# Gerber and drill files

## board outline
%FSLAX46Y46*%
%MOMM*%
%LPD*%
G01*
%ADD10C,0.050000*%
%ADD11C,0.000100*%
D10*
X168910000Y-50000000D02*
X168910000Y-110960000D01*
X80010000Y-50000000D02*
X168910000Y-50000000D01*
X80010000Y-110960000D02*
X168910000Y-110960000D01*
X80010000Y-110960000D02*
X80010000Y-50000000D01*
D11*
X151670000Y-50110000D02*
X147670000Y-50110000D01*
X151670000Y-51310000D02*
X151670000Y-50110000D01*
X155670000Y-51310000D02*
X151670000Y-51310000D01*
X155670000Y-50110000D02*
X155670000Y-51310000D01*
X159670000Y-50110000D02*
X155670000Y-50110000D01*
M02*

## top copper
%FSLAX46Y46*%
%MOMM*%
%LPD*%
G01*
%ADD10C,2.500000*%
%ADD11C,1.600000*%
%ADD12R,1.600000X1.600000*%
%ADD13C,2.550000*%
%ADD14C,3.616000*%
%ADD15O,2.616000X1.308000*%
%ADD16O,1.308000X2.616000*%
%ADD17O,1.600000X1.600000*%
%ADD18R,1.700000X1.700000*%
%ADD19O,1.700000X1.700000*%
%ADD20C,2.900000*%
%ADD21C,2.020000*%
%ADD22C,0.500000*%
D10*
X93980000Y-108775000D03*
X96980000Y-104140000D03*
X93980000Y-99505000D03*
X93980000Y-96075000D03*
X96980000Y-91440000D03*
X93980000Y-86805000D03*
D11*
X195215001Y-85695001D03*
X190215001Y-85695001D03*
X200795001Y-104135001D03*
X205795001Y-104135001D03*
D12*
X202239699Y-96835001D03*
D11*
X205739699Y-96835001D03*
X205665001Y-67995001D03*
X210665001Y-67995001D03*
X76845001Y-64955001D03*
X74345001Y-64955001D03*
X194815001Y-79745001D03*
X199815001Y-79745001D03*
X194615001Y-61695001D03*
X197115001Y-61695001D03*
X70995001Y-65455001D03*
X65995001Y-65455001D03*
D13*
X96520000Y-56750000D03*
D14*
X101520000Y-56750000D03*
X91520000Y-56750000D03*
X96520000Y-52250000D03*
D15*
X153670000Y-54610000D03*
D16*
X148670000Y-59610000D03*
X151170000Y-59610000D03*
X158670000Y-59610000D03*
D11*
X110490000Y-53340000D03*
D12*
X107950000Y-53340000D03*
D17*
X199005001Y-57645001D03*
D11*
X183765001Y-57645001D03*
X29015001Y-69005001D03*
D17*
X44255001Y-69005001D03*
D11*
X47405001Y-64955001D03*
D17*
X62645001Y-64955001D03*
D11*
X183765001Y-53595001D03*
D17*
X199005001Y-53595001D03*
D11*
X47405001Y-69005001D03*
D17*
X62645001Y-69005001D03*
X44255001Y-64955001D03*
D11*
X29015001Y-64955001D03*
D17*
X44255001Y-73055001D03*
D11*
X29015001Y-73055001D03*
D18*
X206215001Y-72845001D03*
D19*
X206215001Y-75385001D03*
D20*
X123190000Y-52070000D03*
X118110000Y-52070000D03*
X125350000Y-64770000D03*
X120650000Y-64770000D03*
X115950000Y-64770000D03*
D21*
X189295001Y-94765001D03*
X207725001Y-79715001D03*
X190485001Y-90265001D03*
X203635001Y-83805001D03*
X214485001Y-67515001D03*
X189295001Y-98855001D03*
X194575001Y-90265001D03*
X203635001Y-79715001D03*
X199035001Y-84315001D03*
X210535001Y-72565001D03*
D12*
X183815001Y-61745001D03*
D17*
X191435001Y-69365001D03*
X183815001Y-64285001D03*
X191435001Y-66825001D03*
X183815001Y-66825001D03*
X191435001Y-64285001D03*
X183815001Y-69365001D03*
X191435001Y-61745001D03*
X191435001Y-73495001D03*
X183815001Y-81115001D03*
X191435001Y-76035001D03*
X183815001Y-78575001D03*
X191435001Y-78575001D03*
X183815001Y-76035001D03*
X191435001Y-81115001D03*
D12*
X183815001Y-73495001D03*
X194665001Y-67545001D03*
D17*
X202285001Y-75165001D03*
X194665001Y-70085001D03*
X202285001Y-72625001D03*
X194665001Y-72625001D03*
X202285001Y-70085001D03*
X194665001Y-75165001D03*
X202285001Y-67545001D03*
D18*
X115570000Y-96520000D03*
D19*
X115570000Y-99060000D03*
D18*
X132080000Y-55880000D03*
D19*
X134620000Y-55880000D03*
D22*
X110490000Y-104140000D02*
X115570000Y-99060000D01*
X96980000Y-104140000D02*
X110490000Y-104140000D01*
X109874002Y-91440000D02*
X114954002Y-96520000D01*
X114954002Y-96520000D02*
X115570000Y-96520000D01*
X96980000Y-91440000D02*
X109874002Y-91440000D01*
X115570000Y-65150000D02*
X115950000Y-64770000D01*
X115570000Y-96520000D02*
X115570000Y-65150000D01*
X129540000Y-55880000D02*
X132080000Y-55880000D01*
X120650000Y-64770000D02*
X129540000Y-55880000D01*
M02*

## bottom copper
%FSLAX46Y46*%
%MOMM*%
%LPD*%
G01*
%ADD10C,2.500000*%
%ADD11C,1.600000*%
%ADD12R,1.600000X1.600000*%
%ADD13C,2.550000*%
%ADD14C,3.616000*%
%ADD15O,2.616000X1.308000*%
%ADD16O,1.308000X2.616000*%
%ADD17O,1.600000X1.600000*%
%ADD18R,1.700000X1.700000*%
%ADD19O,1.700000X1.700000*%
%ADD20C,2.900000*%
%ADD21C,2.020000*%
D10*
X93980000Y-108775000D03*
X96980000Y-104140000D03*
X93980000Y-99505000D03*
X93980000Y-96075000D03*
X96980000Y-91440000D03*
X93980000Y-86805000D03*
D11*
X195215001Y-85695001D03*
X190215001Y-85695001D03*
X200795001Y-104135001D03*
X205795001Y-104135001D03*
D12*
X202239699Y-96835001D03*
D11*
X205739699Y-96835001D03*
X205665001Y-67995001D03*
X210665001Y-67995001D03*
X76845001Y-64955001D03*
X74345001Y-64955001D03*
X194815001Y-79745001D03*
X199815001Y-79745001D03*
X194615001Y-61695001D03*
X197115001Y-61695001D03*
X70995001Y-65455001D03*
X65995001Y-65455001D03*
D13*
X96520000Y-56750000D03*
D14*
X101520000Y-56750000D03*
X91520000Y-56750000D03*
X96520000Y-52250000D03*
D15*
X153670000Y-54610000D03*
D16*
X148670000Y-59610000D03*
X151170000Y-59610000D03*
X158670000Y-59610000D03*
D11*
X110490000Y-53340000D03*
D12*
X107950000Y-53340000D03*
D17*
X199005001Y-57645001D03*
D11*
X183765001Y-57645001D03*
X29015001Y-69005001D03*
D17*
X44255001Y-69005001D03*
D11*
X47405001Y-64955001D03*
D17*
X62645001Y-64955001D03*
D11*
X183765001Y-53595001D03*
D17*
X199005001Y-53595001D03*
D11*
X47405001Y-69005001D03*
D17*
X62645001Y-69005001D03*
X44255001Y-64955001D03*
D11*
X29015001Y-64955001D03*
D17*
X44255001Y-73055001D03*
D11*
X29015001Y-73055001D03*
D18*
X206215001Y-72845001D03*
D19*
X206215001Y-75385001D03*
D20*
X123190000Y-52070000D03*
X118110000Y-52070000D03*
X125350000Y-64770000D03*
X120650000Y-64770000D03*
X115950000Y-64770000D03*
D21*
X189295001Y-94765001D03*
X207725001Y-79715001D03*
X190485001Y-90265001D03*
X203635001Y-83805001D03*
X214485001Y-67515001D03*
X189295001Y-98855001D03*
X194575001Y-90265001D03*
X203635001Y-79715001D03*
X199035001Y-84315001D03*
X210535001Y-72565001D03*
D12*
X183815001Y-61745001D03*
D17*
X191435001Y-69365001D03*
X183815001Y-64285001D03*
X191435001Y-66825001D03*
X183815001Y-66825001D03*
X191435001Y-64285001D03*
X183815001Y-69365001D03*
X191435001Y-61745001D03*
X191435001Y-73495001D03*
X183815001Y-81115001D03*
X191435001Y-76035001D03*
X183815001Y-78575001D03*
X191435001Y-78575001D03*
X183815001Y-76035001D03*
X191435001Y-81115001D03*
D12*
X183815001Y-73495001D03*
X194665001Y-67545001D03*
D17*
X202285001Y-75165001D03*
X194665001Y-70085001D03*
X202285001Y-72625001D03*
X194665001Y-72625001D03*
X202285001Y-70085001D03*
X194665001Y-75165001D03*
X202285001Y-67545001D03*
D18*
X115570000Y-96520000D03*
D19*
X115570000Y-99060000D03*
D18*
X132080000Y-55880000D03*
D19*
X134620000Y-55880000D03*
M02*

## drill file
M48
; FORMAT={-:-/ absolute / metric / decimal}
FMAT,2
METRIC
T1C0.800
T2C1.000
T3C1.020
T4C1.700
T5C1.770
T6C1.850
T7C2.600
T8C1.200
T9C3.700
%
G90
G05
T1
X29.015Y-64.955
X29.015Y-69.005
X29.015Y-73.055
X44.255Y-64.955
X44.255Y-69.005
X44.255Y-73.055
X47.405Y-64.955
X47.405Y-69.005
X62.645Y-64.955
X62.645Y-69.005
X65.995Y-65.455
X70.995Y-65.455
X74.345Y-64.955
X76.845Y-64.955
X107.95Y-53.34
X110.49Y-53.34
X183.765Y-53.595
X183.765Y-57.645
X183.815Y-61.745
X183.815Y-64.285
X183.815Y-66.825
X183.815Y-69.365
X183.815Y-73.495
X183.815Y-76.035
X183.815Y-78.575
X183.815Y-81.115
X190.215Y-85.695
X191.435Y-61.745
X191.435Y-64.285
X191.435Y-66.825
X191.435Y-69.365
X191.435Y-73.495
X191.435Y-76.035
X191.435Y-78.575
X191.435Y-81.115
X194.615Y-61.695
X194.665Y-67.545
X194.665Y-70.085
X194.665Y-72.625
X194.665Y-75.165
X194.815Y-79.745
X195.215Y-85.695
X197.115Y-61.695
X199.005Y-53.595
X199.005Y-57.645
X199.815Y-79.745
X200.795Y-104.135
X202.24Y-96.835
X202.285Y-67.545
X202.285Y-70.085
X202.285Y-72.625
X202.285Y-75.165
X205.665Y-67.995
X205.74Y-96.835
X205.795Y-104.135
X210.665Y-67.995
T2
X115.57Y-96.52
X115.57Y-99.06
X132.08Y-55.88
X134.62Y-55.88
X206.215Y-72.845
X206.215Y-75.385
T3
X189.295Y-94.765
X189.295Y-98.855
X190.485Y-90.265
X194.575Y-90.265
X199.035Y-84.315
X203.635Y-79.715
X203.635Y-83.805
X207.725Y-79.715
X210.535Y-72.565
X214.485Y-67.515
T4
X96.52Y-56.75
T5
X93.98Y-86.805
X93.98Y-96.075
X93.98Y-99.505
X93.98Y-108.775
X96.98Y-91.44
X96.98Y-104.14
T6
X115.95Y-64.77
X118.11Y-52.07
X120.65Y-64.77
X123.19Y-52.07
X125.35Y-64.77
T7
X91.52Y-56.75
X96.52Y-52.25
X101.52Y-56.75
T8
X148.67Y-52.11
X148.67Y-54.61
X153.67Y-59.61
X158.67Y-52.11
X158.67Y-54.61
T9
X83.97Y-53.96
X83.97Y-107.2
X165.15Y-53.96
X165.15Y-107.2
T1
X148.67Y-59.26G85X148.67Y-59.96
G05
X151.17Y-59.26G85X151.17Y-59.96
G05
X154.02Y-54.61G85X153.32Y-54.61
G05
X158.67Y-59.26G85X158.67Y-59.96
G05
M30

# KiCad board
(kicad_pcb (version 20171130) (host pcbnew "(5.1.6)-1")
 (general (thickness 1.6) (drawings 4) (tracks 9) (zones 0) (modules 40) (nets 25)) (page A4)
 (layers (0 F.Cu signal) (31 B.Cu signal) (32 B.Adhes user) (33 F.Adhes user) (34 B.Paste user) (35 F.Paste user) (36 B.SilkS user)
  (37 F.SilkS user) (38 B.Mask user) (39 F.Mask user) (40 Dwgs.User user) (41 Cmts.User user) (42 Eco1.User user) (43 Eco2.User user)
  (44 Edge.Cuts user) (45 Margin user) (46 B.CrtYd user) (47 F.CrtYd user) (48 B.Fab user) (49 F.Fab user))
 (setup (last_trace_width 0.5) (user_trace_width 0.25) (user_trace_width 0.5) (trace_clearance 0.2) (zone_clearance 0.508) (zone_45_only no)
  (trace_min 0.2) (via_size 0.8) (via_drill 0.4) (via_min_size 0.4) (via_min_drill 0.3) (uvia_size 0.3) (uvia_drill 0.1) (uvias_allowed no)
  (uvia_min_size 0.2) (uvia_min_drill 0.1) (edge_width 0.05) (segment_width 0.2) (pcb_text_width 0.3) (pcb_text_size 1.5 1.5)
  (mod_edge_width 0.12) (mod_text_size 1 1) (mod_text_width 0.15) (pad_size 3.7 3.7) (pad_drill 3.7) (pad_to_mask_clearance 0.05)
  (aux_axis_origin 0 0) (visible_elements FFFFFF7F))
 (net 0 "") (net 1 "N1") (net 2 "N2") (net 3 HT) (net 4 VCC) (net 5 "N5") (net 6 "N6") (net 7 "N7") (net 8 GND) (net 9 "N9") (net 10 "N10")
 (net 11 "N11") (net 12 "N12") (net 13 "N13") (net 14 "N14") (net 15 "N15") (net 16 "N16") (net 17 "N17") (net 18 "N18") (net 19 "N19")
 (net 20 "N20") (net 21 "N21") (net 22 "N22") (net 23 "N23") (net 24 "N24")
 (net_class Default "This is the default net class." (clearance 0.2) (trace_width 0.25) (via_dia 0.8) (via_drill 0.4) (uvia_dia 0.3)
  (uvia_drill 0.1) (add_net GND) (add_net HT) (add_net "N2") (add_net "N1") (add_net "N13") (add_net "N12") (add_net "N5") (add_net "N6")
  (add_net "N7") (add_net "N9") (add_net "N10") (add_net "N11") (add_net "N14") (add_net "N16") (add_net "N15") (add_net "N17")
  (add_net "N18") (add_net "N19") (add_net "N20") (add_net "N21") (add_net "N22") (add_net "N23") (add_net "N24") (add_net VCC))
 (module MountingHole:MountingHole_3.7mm (layer F.Cu) (at 83.97 53.96)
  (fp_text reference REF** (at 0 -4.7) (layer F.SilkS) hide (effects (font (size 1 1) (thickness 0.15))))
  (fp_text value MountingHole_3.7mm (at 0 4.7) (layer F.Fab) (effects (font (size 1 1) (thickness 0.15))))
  (pad 1 np_thru_hole circle (at 0 0) (size 3.7 3.7) (drill 3.7) (layers *.Cu *.Mask)))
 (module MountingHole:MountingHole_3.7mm (layer F.Cu) (at 165.15 53.96)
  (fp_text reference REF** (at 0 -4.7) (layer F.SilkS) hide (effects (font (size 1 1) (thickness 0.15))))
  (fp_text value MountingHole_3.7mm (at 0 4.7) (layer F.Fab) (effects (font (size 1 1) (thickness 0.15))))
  (pad 1 np_thru_hole circle (at 0 0) (size 3.7 3.7) (drill 3.7) (layers *.Cu *.Mask)))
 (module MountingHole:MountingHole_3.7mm (layer F.Cu) (at 165.15 107.2)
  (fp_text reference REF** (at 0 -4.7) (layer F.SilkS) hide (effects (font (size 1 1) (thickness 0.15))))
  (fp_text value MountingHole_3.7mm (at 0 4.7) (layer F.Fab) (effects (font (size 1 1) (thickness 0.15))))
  (pad 1 np_thru_hole circle (at 0 0) (size 3.7 3.7) (drill 3.7) (layers *.Cu *.Mask)))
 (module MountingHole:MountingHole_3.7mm (layer F.Cu) (at 83.97 107.2)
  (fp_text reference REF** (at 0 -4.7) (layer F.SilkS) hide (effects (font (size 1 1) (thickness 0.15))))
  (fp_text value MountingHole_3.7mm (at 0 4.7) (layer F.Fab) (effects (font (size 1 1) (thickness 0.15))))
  (pad 1 np_thru_hole circle (at 0 0) (size 3.7 3.7) (drill 3.7) (layers *.Cu *.Mask)))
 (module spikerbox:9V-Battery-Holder (layer F.Cu) (at 93.98 97.79)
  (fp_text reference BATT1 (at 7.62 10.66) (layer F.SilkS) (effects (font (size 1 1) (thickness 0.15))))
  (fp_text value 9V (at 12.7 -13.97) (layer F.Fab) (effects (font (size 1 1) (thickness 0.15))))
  (pad "" thru_hole circle (at 0 10.985) (size 2.5 2.5) (drill 1.77) (layers *.Cu *.Mask))
  (pad 2 thru_hole circle (at 3 6.35) (size 2.5 2.5) (drill 1.77) (layers *.Cu *.Mask) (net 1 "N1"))
  (pad "" thru_hole circle (at 0 1.715) (size 2.5 2.5) (drill 1.77) (layers *.Cu *.Mask))
  (pad "" thru_hole circle (at 0 -1.715) (size 2.5 2.5) (drill 1.77) (layers *.Cu *.Mask))
  (pad 1 thru_hole circle (at 3 -6.35) (size 2.5 2.5) (drill 1.77) (layers *.Cu *.Mask) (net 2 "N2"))
  (pad "" thru_hole circle (at 0 -10.985) (size 2.5 2.5) (drill 1.77) (layers *.Cu *.Mask)))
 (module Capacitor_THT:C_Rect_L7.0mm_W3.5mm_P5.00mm (layer F.Cu) (at 190.215001 85.695001)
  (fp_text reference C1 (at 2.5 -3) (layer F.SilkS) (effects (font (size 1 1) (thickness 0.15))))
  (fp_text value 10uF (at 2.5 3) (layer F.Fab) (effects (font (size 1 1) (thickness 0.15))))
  (pad 2 thru_hole circle (at 5 0) (size 1.6 1.6) (drill 0.8) (layers *.Cu *.Mask) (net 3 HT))
  (pad 1 thru_hole circle (at 0 0) (size 1.6 1.6) (drill 0.8) (layers *.Cu *.Mask) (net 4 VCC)))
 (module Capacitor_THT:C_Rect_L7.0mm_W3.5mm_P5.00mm (layer F.Cu) (at 200.795001 104.135001)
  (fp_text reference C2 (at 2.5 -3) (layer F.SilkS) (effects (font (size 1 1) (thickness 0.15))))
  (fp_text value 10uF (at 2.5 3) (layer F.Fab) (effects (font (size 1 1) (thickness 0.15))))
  (pad 1 thru_hole circle (at 0 0) (size 1.6 1.6) (drill 0.8) (layers *.Cu *.Mask) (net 3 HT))
  (pad 2 thru_hole circle (at 5 0) (size 1.6 1.6) (drill 0.8) (layers *.Cu *.Mask) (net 1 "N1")))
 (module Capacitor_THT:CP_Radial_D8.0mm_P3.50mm (layer F.Cu) (at 202.239699 96.835001)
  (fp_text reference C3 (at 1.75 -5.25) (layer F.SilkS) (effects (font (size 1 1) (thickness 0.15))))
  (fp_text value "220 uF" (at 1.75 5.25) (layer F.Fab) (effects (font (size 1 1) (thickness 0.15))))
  (pad 1 thru_hole rect (at 0 0) (size 1.6 1.6) (drill 0.8) (layers *.Cu *.Mask) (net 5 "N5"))
  (pad 2 thru_hole circle (at 3.5 0) (size 1.6 1.6) (drill 0.8) (layers *.Cu *.Mask) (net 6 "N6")))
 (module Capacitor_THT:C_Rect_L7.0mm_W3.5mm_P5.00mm (layer F.Cu) (at 205.665001 67.995001)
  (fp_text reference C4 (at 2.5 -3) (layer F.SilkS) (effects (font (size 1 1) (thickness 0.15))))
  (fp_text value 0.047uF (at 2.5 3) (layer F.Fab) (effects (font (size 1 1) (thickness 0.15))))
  (pad 1 thru_hole circle (at 0 0) (size 1.6 1.6) (drill 0.8) (layers *.Cu *.Mask) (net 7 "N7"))
  (pad 2 thru_hole circle (at 5 0) (size 1.6 1.6) (drill 0.8) (layers *.Cu *.Mask) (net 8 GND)))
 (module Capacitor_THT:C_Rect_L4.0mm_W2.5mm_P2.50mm (layer F.Cu) (at 74.345001 64.955001)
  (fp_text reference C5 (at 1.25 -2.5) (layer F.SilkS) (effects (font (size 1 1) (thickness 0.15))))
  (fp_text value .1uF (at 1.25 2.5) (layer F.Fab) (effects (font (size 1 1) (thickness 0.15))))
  (pad 2 thru_hole circle (at 2.5 0) (size 1.6 1.6) (drill 0.8) (layers *.Cu *.Mask) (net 8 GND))
  (pad 1 thru_hole circle (at 0 0) (size 1.6 1.6) (drill 0.8) (layers *.Cu *.Mask) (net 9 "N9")))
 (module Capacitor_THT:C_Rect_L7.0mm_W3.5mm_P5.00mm (layer F.Cu) (at 194.815001 79.745001)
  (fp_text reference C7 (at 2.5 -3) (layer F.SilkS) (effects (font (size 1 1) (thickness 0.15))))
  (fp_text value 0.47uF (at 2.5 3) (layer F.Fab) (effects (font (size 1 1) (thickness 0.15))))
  (pad 1 thru_hole circle (at 0 0) (size 1.6 1.6) (drill 0.8) (layers *.Cu *.Mask) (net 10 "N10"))
  (pad 2 thru_hole circle (at 5 0) (size 1.6 1.6) (drill 0.8) (layers *.Cu *.Mask) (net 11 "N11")))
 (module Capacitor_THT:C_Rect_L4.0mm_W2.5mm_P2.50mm (layer F.Cu) (at 194.615001 61.695001)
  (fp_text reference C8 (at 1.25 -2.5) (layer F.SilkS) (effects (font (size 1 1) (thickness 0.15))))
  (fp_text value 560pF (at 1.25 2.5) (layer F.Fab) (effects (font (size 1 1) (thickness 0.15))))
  (pad 1 thru_hole circle (at 0 0) (size 1.6 1.6) (drill 0.8) (layers *.Cu *.Mask) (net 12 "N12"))
  (pad 2 thru_hole circle (at 2.5 0) (size 1.6 1.6) (drill 0.8) (layers *.Cu *.Mask) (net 10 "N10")))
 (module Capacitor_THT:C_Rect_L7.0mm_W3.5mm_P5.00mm (layer F.Cu) (at 65.995001 65.455001)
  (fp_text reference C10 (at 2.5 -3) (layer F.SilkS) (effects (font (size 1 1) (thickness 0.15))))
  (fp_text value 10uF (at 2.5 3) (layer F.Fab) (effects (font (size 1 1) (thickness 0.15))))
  (pad 2 thru_hole circle (at 5 0) (size 1.6 1.6) (drill 0.8) (layers *.Cu *.Mask) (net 12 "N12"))
  (pad 1 thru_hole circle (at 0 0) (size 1.6 1.6) (drill 0.8) (layers *.Cu *.Mask) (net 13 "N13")))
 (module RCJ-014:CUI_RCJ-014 (layer F.Cu) (at 96.52 50.8 270)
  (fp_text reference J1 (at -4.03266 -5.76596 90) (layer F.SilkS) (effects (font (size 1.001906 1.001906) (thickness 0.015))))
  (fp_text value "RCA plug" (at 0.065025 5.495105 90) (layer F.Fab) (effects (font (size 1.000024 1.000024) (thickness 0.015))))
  (pad 2 thru_hole circle (at 5.95 0 270) (size 2.55 2.55) (drill 1.7) (layers *.Cu *.Mask) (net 3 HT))
  (pad 1A thru_hole circle (at 5.95 -5 270) (size 3.616 3.616) (drill 2.6) (layers *.Cu *.Mask) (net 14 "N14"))
  (pad 1B thru_hole circle (at 5.95 5 270) (size 3.616 3.616) (drill 2.6) (layers *.Cu *.Mask) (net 14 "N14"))
  (pad 1C thru_hole circle (at 1.45 0 270) (size 3.616 3.616) (drill 2.6) (layers *.Cu *.Mask) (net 14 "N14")))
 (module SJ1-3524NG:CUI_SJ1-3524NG (layer F.Cu) (at 153.67 54.61 270)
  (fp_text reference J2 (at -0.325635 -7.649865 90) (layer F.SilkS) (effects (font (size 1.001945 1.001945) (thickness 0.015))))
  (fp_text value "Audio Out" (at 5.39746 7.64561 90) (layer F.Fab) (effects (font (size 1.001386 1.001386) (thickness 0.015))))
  (fp_line (start -4.5 2) (end -4.5 6) (layer Edge.Cuts) (width 0.0001))
  (fp_line (start -3.3 2) (end -4.5 2) (layer Edge.Cuts) (width 0.0001))
  (fp_line (start -3.3 -2) (end -3.3 2) (layer Edge.Cuts) (width 0.0001))
  (fp_line (start -4.5 -2) (end -3.3 -2) (layer Edge.Cuts) (width 0.0001))
  (fp_line (start -4.5 -6) (end -4.5 -2) (layer Edge.Cuts) (width 0.0001))
  (pad 1 thru_hole oval (at 0 0 270) (size 1.308 2.616) (drill oval 0.8 1.5) (layers *.Cu *.Mask) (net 8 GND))
  (pad 2 thru_hole oval (at 5 5 270) (size 2.616 1.308) (drill oval 1.5 0.8) (layers *.Cu *.Mask) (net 13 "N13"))
  (pad 4 thru_hole oval (at 5 2.5 270) (size 2.616 1.308) (drill oval 1.5 0.8) (layers *.Cu *.Mask) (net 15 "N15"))
  (pad 3 thru_hole oval (at 5 -5 270) (size 2.616 1.308) (drill oval 1.5 0.8) (layers *.Cu *.Mask) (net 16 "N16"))
  (pad None np_thru_hole circle (at -2.5 -5 270) (size 1.2 1.2) (drill 1.2) (layers *.Cu *.Mask))
  (pad None np_thru_hole circle (at 0 -5 270) (size 1.2 1.2) (drill 1.2) (layers *.Cu *.Mask))
  (pad None np_thru_hole circle (at 5 0 270) (size 1.2 1.2) (drill 1.2) (layers *.Cu *.Mask))
  (pad None np_thru_hole circle (at -2.5 5 270) (size 1.2 1.2) (drill 1.2) (layers *.Cu *.Mask))
  (pad None np_thru_hole circle (at 0 5 270) (size 1.2 1.2) (drill 1.2) (layers *.Cu *.Mask)))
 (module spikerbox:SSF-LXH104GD (layer F.Cu) (at 109.22 53.34 270)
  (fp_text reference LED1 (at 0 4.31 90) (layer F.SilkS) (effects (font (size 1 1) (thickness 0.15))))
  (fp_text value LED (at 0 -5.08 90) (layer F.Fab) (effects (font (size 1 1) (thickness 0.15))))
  (pad 2 thru_hole circle (at 0 -1.27 270) (size 1.6 1.6) (drill 0.8) (layers *.Cu *.Mask) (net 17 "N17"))
  (pad 1 thru_hole rect (at 0 1.27 270) (size 1.6 1.6) (drill 0.8) (layers *.Cu *.Mask) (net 1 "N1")))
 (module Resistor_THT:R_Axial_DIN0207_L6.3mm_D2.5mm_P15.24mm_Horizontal (layer F.Cu) (at 183.765001 57.645001)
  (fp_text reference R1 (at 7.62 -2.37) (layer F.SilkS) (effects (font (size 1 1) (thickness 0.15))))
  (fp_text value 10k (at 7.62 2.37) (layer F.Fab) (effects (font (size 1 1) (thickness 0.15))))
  (pad 2 thru_hole oval (at 15.24 0) (size 1.6 1.6) (drill 0.8) (layers *.Cu *.Mask) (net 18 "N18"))
  (pad 1 thru_hole circle (at 0 0) (size 1.6 1.6) (drill 0.8) (layers *.Cu *.Mask) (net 4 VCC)))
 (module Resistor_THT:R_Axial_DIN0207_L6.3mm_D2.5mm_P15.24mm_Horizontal (layer F.Cu) (at 29.015001 69.005001)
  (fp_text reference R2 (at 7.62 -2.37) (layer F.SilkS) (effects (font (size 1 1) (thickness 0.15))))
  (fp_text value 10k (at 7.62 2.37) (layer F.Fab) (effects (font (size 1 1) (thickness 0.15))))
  (pad 1 thru_hole circle (at 0 0) (size 1.6 1.6) (drill 0.8) (layers *.Cu *.Mask) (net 18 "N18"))
  (pad 2 thru_hole oval (at 15.24 0) (size 1.6 1.6) (drill 0.8) (layers *.Cu *.Mask) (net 1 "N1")))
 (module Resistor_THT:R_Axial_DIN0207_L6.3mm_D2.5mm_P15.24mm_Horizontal (layer F.Cu) (at 47.405001 64.955001)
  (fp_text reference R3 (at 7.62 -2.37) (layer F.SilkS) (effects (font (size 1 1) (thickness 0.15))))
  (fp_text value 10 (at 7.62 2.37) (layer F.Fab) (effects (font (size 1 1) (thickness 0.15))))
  (pad 1 thru_hole circle (at 0 0) (size 1.6 1.6) (drill 0.8) (layers *.Cu *.Mask) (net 5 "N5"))
  (pad 2 thru_hole oval (at 15.24 0) (size 1.6 1.6) (drill 0.8) (layers *.Cu *.Mask) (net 7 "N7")))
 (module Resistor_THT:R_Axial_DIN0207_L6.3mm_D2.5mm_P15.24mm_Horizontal (layer F.Cu) (at 183.765001 53.595001)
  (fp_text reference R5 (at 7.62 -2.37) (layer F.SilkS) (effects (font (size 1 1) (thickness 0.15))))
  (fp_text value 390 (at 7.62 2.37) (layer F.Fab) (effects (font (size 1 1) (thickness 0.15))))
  (pad 1 thru_hole circle (at 0 0) (size 1.6 1.6) (drill 0.8) (layers *.Cu *.Mask) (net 4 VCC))
  (pad 2 thru_hole oval (at 15.24 0) (size 1.6 1.6) (drill 0.8) (layers *.Cu *.Mask) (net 17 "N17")))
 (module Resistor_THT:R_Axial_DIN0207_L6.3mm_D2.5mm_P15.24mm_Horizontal (layer F.Cu) (at 47.405001 69.005001)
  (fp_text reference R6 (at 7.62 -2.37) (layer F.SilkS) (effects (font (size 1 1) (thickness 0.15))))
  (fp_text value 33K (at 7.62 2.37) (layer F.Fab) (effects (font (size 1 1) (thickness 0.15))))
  (pad 1 thru_hole circle (at 0 0) (size 1.6 1.6) (drill 0.8) (layers *.Cu *.Mask) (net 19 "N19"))
  (pad 2 thru_hole oval (at 15.24 0) (size 1.6 1.6) (drill 0.8) (layers *.Cu *.Mask) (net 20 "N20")))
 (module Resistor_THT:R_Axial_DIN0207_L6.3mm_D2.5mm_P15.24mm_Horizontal (layer F.Cu) (at 29.015001 64.955001)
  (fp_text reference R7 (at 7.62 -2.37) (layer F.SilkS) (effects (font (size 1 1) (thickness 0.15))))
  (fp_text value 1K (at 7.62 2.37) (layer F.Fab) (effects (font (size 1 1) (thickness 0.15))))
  (pad 2 thru_hole oval (at 15.24 0) (size 1.6 1.6) (drill 0.8) (layers *.Cu *.Mask) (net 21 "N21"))
  (pad 1 thru_hole circle (at 0 0) (size 1.6 1.6) (drill 0.8) (layers *.Cu *.Mask) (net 11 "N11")))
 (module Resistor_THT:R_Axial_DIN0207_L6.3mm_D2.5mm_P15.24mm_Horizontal (layer F.Cu) (at 29.015001 73.055001)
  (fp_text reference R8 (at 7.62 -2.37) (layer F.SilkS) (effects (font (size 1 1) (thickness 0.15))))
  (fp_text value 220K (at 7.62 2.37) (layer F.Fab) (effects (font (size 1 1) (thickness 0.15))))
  (pad 2 thru_hole oval (at 15.24 0) (size 1.6 1.6) (drill 0.8) (layers *.Cu *.Mask) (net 10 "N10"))
  (pad 1 thru_hole circle (at 0 0) (size 1.6 1.6) (drill 0.8) (layers *.Cu *.Mask) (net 12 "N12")))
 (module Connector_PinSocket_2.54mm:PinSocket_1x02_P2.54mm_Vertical (layer F.Cu) (at 206.215001 72.845001)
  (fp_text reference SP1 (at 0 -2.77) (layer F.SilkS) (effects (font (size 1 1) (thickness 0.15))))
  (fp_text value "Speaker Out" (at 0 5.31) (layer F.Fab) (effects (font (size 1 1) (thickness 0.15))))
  (pad 1 thru_hole rect (at 0 0) (size 1.7 1.7) (drill 1) (layers *.Cu *.Mask) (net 6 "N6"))
  (pad 2 thru_hole oval (at 0 2.54) (size 1.7 1.7) (drill 1) (layers *.Cu *.Mask) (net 8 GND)))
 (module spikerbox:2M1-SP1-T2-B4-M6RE (layer F.Cu) (at 120.65 64.77 270)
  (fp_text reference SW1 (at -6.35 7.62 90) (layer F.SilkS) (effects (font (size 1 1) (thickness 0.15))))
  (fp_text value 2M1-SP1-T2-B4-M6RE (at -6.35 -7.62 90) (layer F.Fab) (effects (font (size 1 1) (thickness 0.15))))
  (pad "" thru_hole circle (at -12.7 -2.54 270) (size 2.9 2.9) (drill 1.85) (layers *.Cu *.Mask))
  (pad "" thru_hole circle (at -12.7 2.54 270) (size 2.9 2.9) (drill 1.85) (layers *.Cu *.Mask))
  (pad 3 thru_hole circle (at 0 -4.7 270) (size 2.9 2.9) (drill 1.85) (layers *.Cu *.Mask) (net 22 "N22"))
  (pad 2 thru_hole circle (at 0 0 270) (size 2.9 2.9) (drill 1.85) (layers *.Cu *.Mask) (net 4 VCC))
  (pad 1 thru_hole circle (at 0 4.7 270) (size 2.9 2.9) (drill 1.85) (layers *.Cu *.Mask) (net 2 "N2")))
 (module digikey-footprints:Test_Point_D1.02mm (layer F.Cu) (at 189.295001 94.765001)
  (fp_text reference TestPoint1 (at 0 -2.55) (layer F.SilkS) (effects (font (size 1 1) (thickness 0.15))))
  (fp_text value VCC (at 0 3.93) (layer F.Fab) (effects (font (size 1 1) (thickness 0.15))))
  (pad 1 thru_hole circle (at 0 0) (size 2.02 2.02) (drill 1.02) (layers *.Cu *.Mask) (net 4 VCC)))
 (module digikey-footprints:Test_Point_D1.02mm (layer F.Cu) (at 207.725001 79.715001)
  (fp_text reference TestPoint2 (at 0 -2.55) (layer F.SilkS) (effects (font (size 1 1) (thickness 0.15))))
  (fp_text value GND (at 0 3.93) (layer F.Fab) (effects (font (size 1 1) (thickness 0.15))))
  (pad 1 thru_hole circle (at 0 0) (size 2.02 2.02) (drill 1.02) (layers *.Cu *.Mask) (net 1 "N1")))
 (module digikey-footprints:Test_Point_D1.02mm (layer F.Cu) (at 190.485001 90.265001)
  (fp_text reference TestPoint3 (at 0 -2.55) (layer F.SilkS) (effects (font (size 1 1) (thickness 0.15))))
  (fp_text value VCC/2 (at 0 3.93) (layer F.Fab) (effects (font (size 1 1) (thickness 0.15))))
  (pad 1 thru_hole circle (at 0 0) (size 2.02 2.02) (drill 1.02) (layers *.Cu *.Mask) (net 3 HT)))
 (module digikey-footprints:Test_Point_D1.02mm (layer F.Cu) (at 203.635001 83.805001)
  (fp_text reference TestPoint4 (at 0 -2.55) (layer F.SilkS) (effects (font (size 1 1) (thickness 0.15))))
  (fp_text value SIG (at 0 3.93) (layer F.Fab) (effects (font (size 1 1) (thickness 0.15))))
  (pad 1 thru_hole circle (at 0 0) (size 2.02 2.02) (drill 1.02) (layers *.Cu *.Mask) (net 3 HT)))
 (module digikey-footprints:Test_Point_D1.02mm (layer F.Cu) (at 214.485001 67.515001)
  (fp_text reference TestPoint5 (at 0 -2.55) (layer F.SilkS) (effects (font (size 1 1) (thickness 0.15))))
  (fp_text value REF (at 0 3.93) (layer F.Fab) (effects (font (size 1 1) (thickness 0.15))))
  (pad 1 thru_hole circle (at 0 0) (size 2.02 2.02) (drill 1.02) (layers *.Cu *.Mask) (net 14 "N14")))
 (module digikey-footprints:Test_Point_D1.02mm (layer F.Cu) (at 189.295001 98.855001)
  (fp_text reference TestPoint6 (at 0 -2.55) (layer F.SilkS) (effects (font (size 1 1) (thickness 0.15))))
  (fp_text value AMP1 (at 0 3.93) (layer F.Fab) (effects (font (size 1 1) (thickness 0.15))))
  (pad 1 thru_hole circle (at 0 0) (size 2.02 2.02) (drill 1.02) (layers *.Cu *.Mask) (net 21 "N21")))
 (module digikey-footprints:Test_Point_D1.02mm (layer F.Cu) (at 194.575001 90.265001)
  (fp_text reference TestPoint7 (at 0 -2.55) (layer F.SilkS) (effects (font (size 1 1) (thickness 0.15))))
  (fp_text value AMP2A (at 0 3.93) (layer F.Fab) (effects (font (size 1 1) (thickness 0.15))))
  (pad 1 thru_hole circle (at 0 0) (size 2.02 2.02) (drill 1.02) (layers *.Cu *.Mask) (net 12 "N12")))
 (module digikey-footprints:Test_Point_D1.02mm (layer F.Cu) (at 203.635001 79.715001)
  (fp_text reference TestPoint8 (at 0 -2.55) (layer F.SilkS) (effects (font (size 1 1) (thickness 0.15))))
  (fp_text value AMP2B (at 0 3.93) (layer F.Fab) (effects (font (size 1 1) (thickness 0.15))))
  (pad 1 thru_hole circle (at 0 0) (size 2.02 2.02) (drill 1.02) (layers *.Cu *.Mask) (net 15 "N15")))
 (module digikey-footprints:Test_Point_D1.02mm (layer F.Cu) (at 199.035001 84.315001)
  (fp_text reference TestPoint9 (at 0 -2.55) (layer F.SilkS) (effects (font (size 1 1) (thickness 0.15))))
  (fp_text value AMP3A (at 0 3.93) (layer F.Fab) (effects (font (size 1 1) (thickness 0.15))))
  (pad 1 thru_hole circle (at 0 0) (size 2.02 2.02) (drill 1.02) (layers *.Cu *.Mask) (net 5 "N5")))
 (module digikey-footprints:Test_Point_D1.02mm (layer F.Cu) (at 210.535001 72.565001)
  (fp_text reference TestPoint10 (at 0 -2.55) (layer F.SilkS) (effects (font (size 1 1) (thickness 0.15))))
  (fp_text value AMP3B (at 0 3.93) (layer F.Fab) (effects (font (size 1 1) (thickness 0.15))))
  (pad 1 thru_hole circle (at 0 0) (size 2.02 2.02) (drill 1.02) (layers *.Cu *.Mask) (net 6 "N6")))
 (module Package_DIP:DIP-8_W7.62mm (layer F.Cu) (at 183.815001 61.745001)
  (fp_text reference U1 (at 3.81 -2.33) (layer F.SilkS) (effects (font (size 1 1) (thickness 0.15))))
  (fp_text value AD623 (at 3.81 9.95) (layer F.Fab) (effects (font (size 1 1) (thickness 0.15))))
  (pad 1 thru_hole rect (at 0 0) (size 1.6 1.6) (drill 0.8) (layers *.Cu *.Mask) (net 20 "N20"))
  (pad 5 thru_hole oval (at 7.62 7.62) (size 1.6 1.6) (drill 0.8) (layers *.Cu *.Mask) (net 3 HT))
  (pad 2 thru_hole oval (at 0 2.54) (size 1.6 1.6) (drill 0.8) (layers *.Cu *.Mask) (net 3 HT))
  (pad 6 thru_hole oval (at 7.62 5.08) (size 1.6 1.6) (drill 0.8) (layers *.Cu *.Mask) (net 21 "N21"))
  (pad 3 thru_hole oval (at 0 5.08) (size 1.6 1.6) (drill 0.8) (layers *.Cu *.Mask) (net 14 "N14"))
  (pad 7 thru_hole oval (at 7.62 2.54) (size 1.6 1.6) (drill 0.8) (layers *.Cu *.Mask) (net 4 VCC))
  (pad 4 thru_hole oval (at 0 7.62) (size 1.6 1.6) (drill 0.8) (layers *.Cu *.Mask) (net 8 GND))
  (pad 8 thru_hole oval (at 7.62 0) (size 1.6 1.6) (drill 0.8) (layers *.Cu *.Mask) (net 19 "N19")))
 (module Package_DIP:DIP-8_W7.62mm (layer F.Cu) (at 183.815001 73.495001)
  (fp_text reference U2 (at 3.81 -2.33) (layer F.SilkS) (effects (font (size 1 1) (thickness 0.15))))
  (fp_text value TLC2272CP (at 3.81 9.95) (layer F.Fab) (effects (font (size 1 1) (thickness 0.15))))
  (pad 8 thru_hole oval (at 7.62 0) (size 1.6 1.6) (drill 0.8) (layers *.Cu *.Mask) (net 4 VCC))
  (pad 4 thru_hole oval (at 0 7.62) (size 1.6 1.6) (drill 0.8) (layers *.Cu *.Mask) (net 1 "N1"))
  (pad 7 thru_hole oval (at 7.62 2.54) (size 1.6 1.6) (drill 0.8) (layers *.Cu *.Mask) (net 12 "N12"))
  (pad 3 thru_hole oval (at 0 5.08) (size 1.6 1.6) (drill 0.8) (layers *.Cu *.Mask) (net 18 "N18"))
  (pad 6 thru_hole oval (at 7.62 5.08) (size 1.6 1.6) (drill 0.8) (layers *.Cu *.Mask) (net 10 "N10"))
  (pad 2 thru_hole oval (at 0 2.54) (size 1.6 1.6) (drill 0.8) (layers *.Cu *.Mask) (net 3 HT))
  (pad 5 thru_hole oval (at 7.62 7.62) (size 1.6 1.6) (drill 0.8) (layers *.Cu *.Mask) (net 3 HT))
  (pad 1 thru_hole rect (at 0 0) (size 1.6 1.6) (drill 0.8) (layers *.Cu *.Mask) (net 3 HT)))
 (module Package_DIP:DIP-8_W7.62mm (layer F.Cu) (at 194.665001 67.545001)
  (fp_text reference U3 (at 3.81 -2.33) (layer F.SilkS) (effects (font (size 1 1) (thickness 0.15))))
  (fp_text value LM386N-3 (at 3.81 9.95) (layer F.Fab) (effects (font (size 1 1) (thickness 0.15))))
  (pad 1 thru_hole rect (at 0 0) (size 1.6 1.6) (drill 0.8) (layers *.Cu *.Mask) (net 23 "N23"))
  (pad 5 thru_hole oval (at 7.62 7.62) (size 1.6 1.6) (drill 0.8) (layers *.Cu *.Mask) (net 5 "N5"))
  (pad 2 thru_hole oval (at 0 2.54) (size 1.6 1.6) (drill 0.8) (layers *.Cu *.Mask) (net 8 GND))
  (pad 6 thru_hole oval (at 7.62 5.08) (size 1.6 1.6) (drill 0.8) (layers *.Cu *.Mask) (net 4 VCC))
  (pad 3 thru_hole oval (at 0 5.08) (size 1.6 1.6) (drill 0.8) (layers *.Cu *.Mask) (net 15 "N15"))
  (pad 7 thru_hole oval (at 7.62 2.54) (size 1.6 1.6) (drill 0.8) (layers *.Cu *.Mask) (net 9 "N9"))
  (pad 4 thru_hole oval (at 0 7.62) (size 1.6 1.6) (drill 0.8) (layers *.Cu *.Mask) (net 8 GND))
  (pad 8 thru_hole oval (at 7.62 0) (size 1.6 1.6) (drill 0.8) (layers *.Cu *.Mask) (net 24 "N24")))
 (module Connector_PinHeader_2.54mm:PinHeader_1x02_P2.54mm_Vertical (layer F.Cu) (at 115.57 96.52)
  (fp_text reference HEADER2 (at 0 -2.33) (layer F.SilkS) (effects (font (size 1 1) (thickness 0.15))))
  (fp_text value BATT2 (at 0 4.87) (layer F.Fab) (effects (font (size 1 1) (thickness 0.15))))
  (pad 1 thru_hole rect (at 0 0) (size 1.7 1.7) (drill 1) (layers *.Cu *.Mask) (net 2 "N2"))
  (pad 2 thru_hole oval (at 0 2.54) (size 1.7 1.7) (drill 1) (layers *.Cu *.Mask) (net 1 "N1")))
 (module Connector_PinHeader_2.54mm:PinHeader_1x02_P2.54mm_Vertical (layer F.Cu) (at 132.08 55.88 90)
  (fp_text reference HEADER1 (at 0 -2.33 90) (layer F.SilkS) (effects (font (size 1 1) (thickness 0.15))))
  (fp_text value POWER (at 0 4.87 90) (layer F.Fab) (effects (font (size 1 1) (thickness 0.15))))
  (pad 1 thru_hole rect (at 0 0 90) (size 1.7 1.7) (drill 1) (layers *.Cu *.Mask) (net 4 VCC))
  (pad 2 thru_hole oval (at 0 2.54 90) (size 1.7 1.7) (drill 1) (layers *.Cu *.Mask) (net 1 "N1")))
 (gr_line (start 168.91 50) (end 168.91 110.96) (layer Edge.Cuts) (width 0.05))
 (gr_line (start 80.01 50) (end 168.91 50) (layer Edge.Cuts) (width 0.05))
 (gr_line (start 80.01 110.96) (end 168.91 110.96) (layer Edge.Cuts) (width 0.05))
 (gr_line (start 80.01 110.96) (end 80.01 50) (layer Edge.Cuts) (width 0.05))
 (segment (start 110.49 104.14) (end 115.57 99.06) (width 0.5) (layer F.Cu) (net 1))
 (segment (start 96.98 104.14) (end 110.49 104.14) (width 0.5) (layer F.Cu) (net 1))
 (segment (start 109.874002 91.44) (end 114.954002 96.52) (width 0.5) (layer F.Cu) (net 2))
 (segment (start 114.954002 96.52) (end 115.57 96.52) (width 0.5) (layer F.Cu) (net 2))
 (segment (start 96.98 91.44) (end 109.874002 91.44) (width 0.5) (layer F.Cu) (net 2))
 (segment (start 115.57 65.15) (end 115.95 64.77) (width 0.5) (layer F.Cu) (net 2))
 (segment (start 115.57 96.52) (end 115.57 65.15) (width 0.5) (layer F.Cu) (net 2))
 (segment (start 129.54 55.88) (end 132.08 55.88) (width 0.5) (layer F.Cu) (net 4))
 (segment (start 120.65 64.77) (end 129.54 55.88) (width 0.5) (layer F.Cu) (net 4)))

